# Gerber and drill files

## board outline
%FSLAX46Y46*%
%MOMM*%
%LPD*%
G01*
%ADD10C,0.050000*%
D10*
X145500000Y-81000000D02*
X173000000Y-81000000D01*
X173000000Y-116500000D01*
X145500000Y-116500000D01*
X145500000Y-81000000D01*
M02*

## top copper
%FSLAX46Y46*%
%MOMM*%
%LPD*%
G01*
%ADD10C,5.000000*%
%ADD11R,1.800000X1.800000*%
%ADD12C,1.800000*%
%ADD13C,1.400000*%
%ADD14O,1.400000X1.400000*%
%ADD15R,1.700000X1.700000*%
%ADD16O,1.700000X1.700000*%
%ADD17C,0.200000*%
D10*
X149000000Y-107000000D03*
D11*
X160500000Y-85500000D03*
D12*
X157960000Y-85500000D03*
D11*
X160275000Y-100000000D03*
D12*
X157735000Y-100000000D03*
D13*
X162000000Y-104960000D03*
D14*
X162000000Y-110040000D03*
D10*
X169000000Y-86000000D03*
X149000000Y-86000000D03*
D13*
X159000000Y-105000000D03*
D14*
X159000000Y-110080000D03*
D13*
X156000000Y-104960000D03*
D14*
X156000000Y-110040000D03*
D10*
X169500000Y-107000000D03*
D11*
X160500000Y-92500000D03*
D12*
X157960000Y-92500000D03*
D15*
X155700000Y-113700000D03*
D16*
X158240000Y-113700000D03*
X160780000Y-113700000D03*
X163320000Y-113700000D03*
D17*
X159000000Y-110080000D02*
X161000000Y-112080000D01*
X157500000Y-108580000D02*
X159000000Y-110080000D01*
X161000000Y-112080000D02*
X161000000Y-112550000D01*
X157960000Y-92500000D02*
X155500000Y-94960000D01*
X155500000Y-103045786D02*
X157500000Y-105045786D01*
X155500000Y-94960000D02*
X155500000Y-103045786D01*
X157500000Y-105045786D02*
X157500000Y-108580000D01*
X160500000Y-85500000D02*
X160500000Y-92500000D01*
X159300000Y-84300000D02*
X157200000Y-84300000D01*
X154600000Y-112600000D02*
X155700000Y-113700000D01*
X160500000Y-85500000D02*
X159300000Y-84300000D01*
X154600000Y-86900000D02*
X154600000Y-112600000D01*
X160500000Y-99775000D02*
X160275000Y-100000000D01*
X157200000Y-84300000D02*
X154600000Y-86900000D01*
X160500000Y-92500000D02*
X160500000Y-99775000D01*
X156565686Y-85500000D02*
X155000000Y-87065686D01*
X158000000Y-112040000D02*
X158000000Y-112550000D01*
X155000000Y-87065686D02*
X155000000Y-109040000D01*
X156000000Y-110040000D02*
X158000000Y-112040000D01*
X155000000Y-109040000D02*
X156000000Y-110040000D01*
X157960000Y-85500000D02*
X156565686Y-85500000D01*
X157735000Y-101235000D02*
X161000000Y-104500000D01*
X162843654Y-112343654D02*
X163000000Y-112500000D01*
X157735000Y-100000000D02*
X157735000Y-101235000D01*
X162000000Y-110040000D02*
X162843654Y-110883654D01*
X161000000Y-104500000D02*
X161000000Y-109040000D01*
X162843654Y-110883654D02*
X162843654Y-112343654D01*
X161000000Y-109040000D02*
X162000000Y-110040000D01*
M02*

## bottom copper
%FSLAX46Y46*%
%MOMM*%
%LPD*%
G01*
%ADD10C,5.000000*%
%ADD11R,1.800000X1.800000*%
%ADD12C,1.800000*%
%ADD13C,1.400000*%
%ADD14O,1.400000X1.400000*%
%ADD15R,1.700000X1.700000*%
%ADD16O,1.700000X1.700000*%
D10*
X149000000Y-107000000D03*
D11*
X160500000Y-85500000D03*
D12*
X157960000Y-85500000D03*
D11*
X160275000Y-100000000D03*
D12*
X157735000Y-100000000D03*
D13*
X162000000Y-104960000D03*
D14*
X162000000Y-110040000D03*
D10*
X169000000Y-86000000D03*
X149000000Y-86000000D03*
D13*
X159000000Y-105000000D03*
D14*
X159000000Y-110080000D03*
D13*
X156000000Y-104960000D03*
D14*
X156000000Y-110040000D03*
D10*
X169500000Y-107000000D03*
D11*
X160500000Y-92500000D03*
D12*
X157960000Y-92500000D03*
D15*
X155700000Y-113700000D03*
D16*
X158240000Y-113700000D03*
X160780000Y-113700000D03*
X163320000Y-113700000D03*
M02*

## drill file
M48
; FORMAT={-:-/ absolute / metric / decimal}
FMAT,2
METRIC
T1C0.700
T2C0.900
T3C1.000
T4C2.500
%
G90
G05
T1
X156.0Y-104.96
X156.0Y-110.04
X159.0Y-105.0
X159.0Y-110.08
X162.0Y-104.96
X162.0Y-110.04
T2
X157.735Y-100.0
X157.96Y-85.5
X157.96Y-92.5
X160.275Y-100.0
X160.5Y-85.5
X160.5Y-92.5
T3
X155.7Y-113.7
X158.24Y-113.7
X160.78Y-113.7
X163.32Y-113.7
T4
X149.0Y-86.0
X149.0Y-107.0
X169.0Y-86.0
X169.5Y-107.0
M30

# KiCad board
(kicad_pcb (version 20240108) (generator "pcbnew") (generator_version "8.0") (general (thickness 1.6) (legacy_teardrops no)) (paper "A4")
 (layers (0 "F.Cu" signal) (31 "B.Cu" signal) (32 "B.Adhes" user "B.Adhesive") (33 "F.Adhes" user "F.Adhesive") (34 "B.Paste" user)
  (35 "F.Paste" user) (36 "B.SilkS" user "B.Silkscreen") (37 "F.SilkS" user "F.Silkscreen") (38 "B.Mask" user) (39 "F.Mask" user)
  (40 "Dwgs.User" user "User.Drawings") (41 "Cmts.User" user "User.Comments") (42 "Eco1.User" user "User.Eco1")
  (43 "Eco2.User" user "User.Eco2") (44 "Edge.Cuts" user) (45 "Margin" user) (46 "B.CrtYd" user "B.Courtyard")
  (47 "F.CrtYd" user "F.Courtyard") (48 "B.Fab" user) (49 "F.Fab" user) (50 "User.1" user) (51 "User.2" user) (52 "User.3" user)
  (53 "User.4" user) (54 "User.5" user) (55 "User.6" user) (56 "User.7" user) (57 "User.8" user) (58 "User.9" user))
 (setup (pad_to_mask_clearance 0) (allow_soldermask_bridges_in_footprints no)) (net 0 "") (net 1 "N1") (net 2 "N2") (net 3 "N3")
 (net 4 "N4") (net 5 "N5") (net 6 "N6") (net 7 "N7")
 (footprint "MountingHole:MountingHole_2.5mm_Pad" (layer "F.Cu") (at 149 107)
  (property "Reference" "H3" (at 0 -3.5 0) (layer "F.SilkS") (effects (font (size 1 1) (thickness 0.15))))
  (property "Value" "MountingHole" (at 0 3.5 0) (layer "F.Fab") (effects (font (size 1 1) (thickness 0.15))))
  (pad "1" thru_hole circle (at 0 0) (size 5 5) (drill 2.5) (layers "*.Cu" "*.Mask") (remove_unused_layers no)))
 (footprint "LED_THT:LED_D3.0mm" (layer "F.Cu") (at 160.5 85.5 180)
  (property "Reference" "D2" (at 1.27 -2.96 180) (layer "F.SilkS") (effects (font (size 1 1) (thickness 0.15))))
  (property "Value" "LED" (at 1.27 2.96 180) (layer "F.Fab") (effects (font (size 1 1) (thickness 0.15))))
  (pad "1" thru_hole rect (at 0 0 180) (size 1.8 1.8) (drill 0.9) (layers "*.Cu" "*.Mask") (remove_unused_layers no) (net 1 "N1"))
  (pad "2" thru_hole circle (at 2.54 0 180) (size 1.8 1.8) (drill 0.9) (layers "*.Cu" "*.Mask") (remove_unused_layers no) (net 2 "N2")))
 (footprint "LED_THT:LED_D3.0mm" (layer "F.Cu") (at 160.275 100 180)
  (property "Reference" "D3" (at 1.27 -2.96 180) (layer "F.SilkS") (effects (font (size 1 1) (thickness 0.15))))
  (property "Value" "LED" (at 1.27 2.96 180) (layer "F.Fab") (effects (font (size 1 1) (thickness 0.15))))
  (pad "1" thru_hole rect (at 0 0 180) (size 1.8 1.8) (drill 0.9) (layers "*.Cu" "*.Mask") (remove_unused_layers no) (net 1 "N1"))
  (pad "2" thru_hole circle (at 2.54 0 180) (size 1.8 1.8) (drill 0.9) (layers "*.Cu" "*.Mask") (remove_unused_layers no) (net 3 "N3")))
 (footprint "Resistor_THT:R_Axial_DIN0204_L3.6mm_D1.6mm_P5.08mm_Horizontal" (layer "F.Cu") (at 162 104.96 -90)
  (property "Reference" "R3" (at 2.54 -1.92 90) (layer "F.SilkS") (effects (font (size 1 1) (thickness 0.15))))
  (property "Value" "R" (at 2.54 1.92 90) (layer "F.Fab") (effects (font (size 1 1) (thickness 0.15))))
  (pad "1" thru_hole circle (at 0 0 270) (size 1.4 1.4) (drill 0.7) (layers "*.Cu" "*.Mask") (remove_unused_layers no) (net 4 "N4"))
  (pad "2" thru_hole oval (at 5.08 0 270) (size 1.4 1.4) (drill 0.7) (layers "*.Cu" "*.Mask") (remove_unused_layers no) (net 3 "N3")))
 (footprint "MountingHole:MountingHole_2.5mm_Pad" (layer "F.Cu") (at 169 86)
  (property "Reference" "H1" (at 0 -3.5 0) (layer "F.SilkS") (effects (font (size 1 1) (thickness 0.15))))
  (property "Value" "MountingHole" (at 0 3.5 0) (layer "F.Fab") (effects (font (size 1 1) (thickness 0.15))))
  (pad "1" thru_hole circle (at 0 0) (size 5 5) (drill 2.5) (layers "*.Cu" "*.Mask") (remove_unused_layers no)))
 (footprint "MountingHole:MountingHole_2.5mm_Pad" (layer "F.Cu") (at 149 86)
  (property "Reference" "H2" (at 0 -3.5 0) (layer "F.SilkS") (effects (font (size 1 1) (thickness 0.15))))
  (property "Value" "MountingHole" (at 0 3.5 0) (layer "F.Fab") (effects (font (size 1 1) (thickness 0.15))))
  (pad "1" thru_hole circle (at 0 0) (size 5 5) (drill 2.5) (layers "*.Cu" "*.Mask") (remove_unused_layers no)))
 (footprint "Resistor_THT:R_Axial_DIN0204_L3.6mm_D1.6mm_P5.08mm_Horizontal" (layer "F.Cu") (at 159 105 -90)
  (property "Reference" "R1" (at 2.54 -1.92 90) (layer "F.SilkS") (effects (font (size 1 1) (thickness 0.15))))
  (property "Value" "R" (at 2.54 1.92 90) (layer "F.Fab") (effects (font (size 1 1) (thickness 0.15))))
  (pad "1" thru_hole circle (at 0 0 270) (size 1.4 1.4) (drill 0.7) (layers "*.Cu" "*.Mask") (remove_unused_layers no) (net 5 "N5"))
  (pad "2" thru_hole oval (at 5.08 0 270) (size 1.4 1.4) (drill 0.7) (layers "*.Cu" "*.Mask") (remove_unused_layers no) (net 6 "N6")))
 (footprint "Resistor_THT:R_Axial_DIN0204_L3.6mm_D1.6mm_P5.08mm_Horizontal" (layer "F.Cu") (at 156 104.96 -90)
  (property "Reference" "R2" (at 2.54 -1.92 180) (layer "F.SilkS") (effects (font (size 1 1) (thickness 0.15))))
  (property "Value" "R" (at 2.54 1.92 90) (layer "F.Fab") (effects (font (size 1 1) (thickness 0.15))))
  (pad "1" thru_hole circle (at 0 0 270) (size 1.4 1.4) (drill 0.7) (layers "*.Cu" "*.Mask") (remove_unused_layers no) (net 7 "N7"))
  (pad "2" thru_hole oval (at 5.08 0 270) (size 1.4 1.4) (drill 0.7) (layers "*.Cu" "*.Mask") (remove_unused_layers no) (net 2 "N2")))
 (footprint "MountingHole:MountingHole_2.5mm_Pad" (layer "F.Cu") (at 169.5 107)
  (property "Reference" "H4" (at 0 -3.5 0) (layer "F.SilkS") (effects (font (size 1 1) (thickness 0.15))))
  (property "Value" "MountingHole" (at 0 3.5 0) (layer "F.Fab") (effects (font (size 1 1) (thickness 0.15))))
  (pad "1" thru_hole circle (at 0 0) (size 5 5) (drill 2.5) (layers "*.Cu" "*.Mask") (remove_unused_layers no)))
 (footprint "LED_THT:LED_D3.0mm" (layer "F.Cu") (at 160.5 92.5 180)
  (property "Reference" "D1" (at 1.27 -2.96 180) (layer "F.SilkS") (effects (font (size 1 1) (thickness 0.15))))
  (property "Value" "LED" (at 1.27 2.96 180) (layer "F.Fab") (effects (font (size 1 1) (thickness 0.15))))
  (pad "1" thru_hole rect (at 0 0 180) (size 1.8 1.8) (drill 0.9) (layers "*.Cu" "*.Mask") (remove_unused_layers no) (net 1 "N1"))
  (pad "2" thru_hole circle (at 2.54 0 180) (size 1.8 1.8) (drill 0.9) (layers "*.Cu" "*.Mask") (remove_unused_layers no) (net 6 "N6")))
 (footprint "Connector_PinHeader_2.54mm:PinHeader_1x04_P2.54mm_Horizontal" (layer "B.Cu") (at 155.7 113.7 -90)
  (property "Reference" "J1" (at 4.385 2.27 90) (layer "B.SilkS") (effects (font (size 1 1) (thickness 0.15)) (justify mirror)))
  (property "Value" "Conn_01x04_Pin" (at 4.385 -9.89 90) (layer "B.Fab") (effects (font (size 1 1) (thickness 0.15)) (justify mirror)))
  (pad "1" thru_hole rect (at 0 0 270) (size 1.7 1.7) (drill 1) (layers "*.Cu" "*.Mask") (remove_unused_layers no) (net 1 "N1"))
  (pad "2" thru_hole oval (at 0 -2.54 270) (size 1.7 1.7) (drill 1) (layers "*.Cu" "*.Mask") (remove_unused_layers no) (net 5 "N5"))
  (pad "3" thru_hole oval (at 0 -5.08 270) (size 1.7 1.7) (drill 1) (layers "*.Cu" "*.Mask") (remove_unused_layers no) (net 7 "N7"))
  (pad "4" thru_hole oval (at 0 -7.62 270) (size 1.7 1.7) (drill 1) (layers "*.Cu" "*.Mask") (remove_unused_layers no) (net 4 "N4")))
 (gr_rect (start 145.5 81) (end 173 116.5) (stroke (width 0.05) (type default)) (fill none) (layer "Edge.Cuts"))
 (segment (start 159 110.08) (end 161 112.08) (width 0.2) (layer "F.Cu") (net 6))
 (segment (start 157.5 108.58) (end 159 110.08) (width 0.2) (layer "F.Cu") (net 6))
 (segment (start 161 112.08) (end 161 112.55) (width 0.2) (layer "F.Cu") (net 6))
 (segment (start 157.96 92.5) (end 155.5 94.96) (width 0.2) (layer "F.Cu") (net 6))
 (segment (start 155.5 103.045786) (end 157.5 105.045786) (width 0.2) (layer "F.Cu") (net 6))
 (segment (start 155.5 94.96) (end 155.5 103.045786) (width 0.2) (layer "F.Cu") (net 6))
 (segment (start 157.5 105.045786) (end 157.5 108.58) (width 0.2) (layer "F.Cu") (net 6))
 (segment (start 160.5 85.5) (end 160.5 92.5) (width 0.2) (layer "F.Cu") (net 1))
 (segment (start 159.3 84.3) (end 157.2 84.3) (width 0.2) (layer "F.Cu") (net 1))
 (segment (start 154.6 112.6) (end 155.7 113.7) (width 0.2) (layer "F.Cu") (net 1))
 (segment (start 160.5 85.5) (end 159.3 84.3) (width 0.2) (layer "F.Cu") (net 1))
 (segment (start 154.6 86.9) (end 154.6 112.6) (width 0.2) (layer "F.Cu") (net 1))
 (segment (start 160.5 99.775) (end 160.275 100) (width 0.2) (layer "F.Cu") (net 1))
 (segment (start 157.2 84.3) (end 154.6 86.9) (width 0.2) (layer "F.Cu") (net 1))
 (segment (start 160.5 92.5) (end 160.5 99.775) (width 0.2) (layer "F.Cu") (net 1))
 (segment (start 156.565686 85.5) (end 155 87.065686) (width 0.2) (layer "F.Cu") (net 2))
 (segment (start 158 112.04) (end 158 112.55) (width 0.2) (layer "F.Cu") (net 2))
 (segment (start 155 87.065686) (end 155 109.04) (width 0.2) (layer "F.Cu") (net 2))
 (segment (start 156 110.04) (end 158 112.04) (width 0.2) (layer "F.Cu") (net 2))
 (segment (start 155 109.04) (end 156 110.04) (width 0.2) (layer "F.Cu") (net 2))
 (segment (start 157.96 85.5) (end 156.565686 85.5) (width 0.2) (layer "F.Cu") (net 2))
 (segment (start 157.735 101.235) (end 161 104.5) (width 0.2) (layer "F.Cu") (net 3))
 (segment (start 162.843654 112.343654) (end 163 112.5) (width 0.2) (layer "F.Cu") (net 3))
 (segment (start 157.735 100) (end 157.735 101.235) (width 0.2) (layer "F.Cu") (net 3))
 (segment (start 162 110.04) (end 162.843654 110.883654) (width 0.2) (layer "F.Cu") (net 3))
 (segment (start 161 104.5) (end 161 109.04) (width 0.2) (layer "F.Cu") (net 3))
 (segment (start 162.843654 110.883654) (end 162.843654 112.343654) (width 0.2) (layer "F.Cu") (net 3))
 (segment (start 161 109.04) (end 162 110.04) (width 0.2) (layer "F.Cu") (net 3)))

